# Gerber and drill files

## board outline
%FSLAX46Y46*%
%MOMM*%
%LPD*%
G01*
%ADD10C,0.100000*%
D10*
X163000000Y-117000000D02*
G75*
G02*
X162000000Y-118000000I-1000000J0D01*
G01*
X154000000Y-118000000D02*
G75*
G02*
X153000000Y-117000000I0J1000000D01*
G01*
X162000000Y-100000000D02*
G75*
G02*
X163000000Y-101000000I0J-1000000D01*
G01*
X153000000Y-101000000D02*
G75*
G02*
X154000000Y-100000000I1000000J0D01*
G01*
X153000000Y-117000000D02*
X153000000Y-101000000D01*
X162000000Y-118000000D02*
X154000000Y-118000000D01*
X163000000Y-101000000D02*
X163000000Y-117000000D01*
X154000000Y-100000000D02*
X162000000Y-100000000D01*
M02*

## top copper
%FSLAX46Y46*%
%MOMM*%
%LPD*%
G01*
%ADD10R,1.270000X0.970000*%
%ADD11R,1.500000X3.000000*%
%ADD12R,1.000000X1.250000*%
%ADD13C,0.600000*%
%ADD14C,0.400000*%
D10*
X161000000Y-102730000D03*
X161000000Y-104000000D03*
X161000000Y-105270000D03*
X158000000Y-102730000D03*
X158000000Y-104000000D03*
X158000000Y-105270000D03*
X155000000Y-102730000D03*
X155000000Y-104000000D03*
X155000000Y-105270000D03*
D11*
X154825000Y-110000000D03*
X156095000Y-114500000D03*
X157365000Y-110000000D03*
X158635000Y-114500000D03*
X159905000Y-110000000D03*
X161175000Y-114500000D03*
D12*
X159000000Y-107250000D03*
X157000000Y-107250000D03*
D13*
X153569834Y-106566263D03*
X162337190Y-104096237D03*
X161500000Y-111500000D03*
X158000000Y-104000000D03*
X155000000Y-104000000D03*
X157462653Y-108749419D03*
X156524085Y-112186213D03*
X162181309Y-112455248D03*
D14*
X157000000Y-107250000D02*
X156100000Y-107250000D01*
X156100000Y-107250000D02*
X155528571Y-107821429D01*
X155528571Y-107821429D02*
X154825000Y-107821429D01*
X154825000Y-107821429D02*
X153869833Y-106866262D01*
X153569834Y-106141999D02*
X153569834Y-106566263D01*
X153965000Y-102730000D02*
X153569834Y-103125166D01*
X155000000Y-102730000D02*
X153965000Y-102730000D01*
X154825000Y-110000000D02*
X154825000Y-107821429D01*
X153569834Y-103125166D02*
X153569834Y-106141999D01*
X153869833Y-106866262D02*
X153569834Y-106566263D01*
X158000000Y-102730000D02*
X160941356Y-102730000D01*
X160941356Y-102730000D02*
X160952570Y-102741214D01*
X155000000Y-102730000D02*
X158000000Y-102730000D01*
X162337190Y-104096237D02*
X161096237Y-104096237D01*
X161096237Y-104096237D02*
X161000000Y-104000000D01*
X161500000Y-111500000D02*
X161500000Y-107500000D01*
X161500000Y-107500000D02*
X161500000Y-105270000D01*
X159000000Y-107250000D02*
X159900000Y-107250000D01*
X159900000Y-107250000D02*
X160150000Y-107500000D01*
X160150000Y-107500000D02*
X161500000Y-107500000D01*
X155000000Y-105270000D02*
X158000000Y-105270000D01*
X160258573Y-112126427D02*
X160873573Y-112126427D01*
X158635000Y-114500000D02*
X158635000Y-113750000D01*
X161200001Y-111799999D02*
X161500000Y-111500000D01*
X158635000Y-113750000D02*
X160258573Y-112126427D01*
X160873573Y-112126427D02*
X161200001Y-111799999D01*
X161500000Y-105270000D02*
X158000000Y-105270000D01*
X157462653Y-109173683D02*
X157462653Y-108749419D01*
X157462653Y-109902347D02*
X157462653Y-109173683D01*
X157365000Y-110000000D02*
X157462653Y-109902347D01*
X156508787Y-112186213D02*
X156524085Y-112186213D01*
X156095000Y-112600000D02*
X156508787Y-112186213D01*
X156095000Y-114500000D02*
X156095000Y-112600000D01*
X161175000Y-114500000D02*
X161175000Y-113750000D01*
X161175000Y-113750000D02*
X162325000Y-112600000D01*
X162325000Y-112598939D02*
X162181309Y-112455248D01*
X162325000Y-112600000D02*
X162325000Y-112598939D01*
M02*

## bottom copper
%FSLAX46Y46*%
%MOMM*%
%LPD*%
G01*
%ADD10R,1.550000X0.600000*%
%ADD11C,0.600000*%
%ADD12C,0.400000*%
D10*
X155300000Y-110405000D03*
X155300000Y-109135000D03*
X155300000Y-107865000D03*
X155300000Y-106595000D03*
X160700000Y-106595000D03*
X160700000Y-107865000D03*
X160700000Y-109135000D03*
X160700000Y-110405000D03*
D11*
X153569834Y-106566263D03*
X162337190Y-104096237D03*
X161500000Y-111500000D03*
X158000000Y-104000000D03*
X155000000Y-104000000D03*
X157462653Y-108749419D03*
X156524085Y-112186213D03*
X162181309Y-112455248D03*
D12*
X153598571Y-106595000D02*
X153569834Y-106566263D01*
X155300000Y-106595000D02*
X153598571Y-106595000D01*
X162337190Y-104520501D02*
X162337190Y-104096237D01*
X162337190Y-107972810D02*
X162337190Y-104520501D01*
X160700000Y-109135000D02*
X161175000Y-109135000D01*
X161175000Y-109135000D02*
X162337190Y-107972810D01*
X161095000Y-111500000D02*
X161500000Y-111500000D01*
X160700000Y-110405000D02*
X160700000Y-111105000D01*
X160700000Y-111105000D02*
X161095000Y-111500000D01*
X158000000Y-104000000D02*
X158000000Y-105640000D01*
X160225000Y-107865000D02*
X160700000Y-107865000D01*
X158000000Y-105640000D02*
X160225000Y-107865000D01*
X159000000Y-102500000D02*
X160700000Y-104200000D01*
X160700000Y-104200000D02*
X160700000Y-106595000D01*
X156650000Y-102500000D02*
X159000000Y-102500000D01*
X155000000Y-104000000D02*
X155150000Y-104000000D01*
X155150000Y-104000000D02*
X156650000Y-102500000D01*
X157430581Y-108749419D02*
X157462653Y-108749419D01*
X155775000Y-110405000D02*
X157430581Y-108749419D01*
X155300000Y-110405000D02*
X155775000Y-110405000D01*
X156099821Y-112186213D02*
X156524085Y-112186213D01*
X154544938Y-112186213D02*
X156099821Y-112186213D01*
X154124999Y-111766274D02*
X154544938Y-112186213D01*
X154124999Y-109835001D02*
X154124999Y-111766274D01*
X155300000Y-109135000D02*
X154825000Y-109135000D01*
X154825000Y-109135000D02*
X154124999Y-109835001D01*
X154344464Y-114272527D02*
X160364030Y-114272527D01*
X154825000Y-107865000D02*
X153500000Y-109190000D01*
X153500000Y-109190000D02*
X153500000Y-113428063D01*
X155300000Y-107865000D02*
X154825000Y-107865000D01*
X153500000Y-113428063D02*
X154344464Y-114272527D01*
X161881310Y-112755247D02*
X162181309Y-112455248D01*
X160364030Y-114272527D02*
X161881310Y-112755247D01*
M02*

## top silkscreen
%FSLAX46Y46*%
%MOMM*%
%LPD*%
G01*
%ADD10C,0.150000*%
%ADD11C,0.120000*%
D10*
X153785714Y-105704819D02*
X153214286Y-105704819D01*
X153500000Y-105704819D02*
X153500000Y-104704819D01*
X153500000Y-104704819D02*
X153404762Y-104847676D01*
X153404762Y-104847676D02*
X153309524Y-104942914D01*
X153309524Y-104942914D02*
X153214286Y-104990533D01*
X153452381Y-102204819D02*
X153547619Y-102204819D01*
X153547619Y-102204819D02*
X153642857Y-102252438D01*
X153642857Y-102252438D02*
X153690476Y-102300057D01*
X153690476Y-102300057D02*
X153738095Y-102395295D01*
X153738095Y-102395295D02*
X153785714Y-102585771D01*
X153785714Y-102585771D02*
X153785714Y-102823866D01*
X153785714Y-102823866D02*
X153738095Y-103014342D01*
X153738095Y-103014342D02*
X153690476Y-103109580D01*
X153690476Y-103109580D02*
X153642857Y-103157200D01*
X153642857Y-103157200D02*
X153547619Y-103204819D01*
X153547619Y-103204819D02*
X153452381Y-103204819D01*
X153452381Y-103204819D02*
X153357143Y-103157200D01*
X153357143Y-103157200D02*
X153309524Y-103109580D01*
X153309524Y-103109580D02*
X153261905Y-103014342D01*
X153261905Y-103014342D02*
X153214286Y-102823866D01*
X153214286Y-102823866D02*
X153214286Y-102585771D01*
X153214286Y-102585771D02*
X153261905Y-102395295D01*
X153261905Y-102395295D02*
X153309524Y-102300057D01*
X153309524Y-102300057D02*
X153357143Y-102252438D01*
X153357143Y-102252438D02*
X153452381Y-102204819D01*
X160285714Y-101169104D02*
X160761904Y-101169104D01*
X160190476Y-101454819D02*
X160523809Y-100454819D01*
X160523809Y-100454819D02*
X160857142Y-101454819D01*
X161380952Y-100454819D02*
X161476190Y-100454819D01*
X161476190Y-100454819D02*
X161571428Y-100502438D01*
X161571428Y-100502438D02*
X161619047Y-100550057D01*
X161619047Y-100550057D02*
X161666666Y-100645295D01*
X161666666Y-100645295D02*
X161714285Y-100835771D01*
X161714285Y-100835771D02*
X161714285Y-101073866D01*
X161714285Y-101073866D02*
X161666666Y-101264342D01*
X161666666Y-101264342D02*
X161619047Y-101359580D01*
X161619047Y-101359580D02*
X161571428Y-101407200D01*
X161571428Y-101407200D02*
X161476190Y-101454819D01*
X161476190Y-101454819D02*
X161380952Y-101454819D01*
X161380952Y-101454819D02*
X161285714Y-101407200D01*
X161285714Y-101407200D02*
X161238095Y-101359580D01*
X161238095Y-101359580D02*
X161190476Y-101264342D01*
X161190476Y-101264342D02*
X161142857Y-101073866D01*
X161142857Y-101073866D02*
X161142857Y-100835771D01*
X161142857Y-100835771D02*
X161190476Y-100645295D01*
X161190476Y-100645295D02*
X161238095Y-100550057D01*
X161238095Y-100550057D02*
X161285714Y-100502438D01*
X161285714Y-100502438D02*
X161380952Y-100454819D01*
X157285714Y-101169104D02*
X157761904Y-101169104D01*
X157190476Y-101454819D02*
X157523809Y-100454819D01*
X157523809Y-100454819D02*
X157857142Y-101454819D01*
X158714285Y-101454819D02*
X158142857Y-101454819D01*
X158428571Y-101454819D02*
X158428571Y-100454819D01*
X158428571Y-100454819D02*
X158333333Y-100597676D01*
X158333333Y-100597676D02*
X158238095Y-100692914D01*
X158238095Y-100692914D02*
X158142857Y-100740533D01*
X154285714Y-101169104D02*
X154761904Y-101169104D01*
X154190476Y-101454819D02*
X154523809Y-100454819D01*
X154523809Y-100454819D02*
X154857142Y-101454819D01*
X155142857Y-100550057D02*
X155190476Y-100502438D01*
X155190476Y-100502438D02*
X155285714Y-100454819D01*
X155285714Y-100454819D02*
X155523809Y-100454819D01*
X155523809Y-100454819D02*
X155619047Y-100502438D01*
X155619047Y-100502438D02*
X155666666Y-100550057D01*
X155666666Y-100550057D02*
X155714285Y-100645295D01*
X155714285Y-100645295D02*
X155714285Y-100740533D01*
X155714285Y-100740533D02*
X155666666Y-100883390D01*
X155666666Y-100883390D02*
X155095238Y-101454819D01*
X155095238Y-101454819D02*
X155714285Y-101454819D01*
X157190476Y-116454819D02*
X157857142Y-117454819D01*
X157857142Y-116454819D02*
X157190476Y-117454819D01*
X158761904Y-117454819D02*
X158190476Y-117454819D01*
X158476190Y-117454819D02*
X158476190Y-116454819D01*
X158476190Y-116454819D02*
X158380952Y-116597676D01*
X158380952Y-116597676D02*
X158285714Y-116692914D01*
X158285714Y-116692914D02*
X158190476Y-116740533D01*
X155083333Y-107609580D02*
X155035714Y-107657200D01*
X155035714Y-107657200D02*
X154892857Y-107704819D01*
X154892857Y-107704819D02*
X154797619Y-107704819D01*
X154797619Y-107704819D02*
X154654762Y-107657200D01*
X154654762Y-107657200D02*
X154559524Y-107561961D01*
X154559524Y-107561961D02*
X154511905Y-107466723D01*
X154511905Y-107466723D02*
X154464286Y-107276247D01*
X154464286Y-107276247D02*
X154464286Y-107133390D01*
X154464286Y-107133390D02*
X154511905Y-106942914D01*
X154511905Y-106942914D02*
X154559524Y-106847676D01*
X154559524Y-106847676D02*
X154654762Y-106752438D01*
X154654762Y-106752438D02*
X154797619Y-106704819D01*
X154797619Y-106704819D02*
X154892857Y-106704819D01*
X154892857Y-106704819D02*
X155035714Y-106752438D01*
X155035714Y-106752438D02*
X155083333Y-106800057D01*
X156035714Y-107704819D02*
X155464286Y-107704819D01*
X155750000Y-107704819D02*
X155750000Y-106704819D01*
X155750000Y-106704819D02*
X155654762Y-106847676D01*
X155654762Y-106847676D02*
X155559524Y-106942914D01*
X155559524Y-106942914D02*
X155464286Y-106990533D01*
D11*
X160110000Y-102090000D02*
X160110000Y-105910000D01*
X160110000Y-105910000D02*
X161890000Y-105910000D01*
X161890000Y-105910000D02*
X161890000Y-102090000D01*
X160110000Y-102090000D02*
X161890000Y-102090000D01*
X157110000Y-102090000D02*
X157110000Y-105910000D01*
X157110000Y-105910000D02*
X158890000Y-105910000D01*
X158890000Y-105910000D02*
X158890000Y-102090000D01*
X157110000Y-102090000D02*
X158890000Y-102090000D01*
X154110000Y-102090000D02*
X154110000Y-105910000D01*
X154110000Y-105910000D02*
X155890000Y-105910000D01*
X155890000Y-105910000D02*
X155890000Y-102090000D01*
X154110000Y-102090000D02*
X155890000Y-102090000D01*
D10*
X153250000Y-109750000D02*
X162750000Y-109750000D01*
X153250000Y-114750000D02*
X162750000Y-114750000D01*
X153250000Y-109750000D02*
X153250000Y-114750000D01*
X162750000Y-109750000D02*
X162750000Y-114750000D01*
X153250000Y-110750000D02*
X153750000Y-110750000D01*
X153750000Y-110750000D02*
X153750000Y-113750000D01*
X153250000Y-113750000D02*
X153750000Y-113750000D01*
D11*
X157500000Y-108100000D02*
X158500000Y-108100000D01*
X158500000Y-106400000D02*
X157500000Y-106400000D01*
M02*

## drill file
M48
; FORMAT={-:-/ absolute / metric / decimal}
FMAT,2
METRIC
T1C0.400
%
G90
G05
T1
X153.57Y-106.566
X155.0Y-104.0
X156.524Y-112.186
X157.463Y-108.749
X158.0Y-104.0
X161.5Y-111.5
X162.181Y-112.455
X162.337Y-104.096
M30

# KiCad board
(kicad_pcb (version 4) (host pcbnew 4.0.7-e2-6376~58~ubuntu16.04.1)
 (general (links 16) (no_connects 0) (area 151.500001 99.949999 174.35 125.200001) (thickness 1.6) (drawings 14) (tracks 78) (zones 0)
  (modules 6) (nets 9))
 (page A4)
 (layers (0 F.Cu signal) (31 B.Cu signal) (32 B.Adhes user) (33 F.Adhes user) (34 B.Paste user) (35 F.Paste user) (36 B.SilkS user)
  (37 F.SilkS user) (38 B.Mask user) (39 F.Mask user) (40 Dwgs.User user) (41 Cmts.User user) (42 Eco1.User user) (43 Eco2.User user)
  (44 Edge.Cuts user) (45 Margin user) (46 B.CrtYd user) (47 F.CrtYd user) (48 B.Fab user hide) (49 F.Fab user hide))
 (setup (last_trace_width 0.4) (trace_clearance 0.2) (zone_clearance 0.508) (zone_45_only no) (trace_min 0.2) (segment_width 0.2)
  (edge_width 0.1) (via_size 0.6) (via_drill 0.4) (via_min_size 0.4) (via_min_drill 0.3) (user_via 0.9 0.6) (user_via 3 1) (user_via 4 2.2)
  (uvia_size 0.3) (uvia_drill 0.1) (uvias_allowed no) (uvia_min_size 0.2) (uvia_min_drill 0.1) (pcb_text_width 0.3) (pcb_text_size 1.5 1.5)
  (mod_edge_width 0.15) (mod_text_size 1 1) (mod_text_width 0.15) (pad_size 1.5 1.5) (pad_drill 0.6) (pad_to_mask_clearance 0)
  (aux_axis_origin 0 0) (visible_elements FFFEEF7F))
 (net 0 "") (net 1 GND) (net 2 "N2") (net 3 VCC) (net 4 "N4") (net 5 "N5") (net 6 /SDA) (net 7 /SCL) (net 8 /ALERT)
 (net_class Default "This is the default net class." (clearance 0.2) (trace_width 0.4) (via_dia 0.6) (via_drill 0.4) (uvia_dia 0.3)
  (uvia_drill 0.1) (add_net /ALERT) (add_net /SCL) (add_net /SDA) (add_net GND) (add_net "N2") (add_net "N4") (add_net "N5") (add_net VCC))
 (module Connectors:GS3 (layer F.Cu) (at 161 104)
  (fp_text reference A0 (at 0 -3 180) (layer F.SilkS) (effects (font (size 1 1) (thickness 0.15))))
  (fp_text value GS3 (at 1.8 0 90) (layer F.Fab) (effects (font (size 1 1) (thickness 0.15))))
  (fp_line (start -0.89 -1.91) (end -0.89 1.91) (layer F.SilkS) (width 0.12))
  (fp_line (start -0.89 1.91) (end 0.89 1.91) (layer F.SilkS) (width 0.12))
  (fp_line (start 0.89 1.91) (end 0.89 -1.91) (layer F.SilkS) (width 0.12))
  (fp_line (start -0.89 -1.91) (end 0.89 -1.91) (layer F.SilkS) (width 0.12))
  (pad 1 smd rect (at 0 -1.27) (size 1.27 0.97) (layers F.Cu F.Paste F.Mask) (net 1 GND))
  (pad 2 smd rect (at 0 0) (size 1.27 0.97) (layers F.Cu F.Paste F.Mask) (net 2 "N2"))
  (pad 3 smd rect (at 0 1.27) (size 1.27 0.97) (layers F.Cu F.Paste F.Mask) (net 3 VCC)))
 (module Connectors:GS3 (layer F.Cu) (at 158 104)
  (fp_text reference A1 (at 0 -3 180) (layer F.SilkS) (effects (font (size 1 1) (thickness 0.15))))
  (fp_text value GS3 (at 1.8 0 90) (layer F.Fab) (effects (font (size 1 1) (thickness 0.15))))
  (fp_line (start -0.89 -1.91) (end -0.89 1.91) (layer F.SilkS) (width 0.12))
  (fp_line (start -0.89 1.91) (end 0.89 1.91) (layer F.SilkS) (width 0.12))
  (fp_line (start 0.89 1.91) (end 0.89 -1.91) (layer F.SilkS) (width 0.12))
  (fp_line (start -0.89 -1.91) (end 0.89 -1.91) (layer F.SilkS) (width 0.12))
  (pad 1 smd rect (at 0 -1.27) (size 1.27 0.97) (layers F.Cu F.Paste F.Mask) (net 1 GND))
  (pad 2 smd rect (at 0 0) (size 1.27 0.97) (layers F.Cu F.Paste F.Mask) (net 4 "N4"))
  (pad 3 smd rect (at 0 1.27) (size 1.27 0.97) (layers F.Cu F.Paste F.Mask) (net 3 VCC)))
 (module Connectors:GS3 (layer F.Cu) (at 155 104)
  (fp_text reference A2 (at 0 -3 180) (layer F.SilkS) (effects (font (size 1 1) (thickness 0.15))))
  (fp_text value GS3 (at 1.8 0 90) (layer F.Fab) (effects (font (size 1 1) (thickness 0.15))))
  (fp_line (start -0.89 -1.91) (end -0.89 1.91) (layer F.SilkS) (width 0.12))
  (fp_line (start -0.89 1.91) (end 0.89 1.91) (layer F.SilkS) (width 0.12))
  (fp_line (start 0.89 1.91) (end 0.89 -1.91) (layer F.SilkS) (width 0.12))
  (fp_line (start -0.89 -1.91) (end 0.89 -1.91) (layer F.SilkS) (width 0.12))
  (pad 1 smd rect (at 0 -1.27) (size 1.27 0.97) (layers F.Cu F.Paste F.Mask) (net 1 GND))
  (pad 2 smd rect (at 0 0) (size 1.27 0.97) (layers F.Cu F.Paste F.Mask) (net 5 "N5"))
  (pad 3 smd rect (at 0 1.27) (size 1.27 0.97) (layers F.Cu F.Paste F.Mask) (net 3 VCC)))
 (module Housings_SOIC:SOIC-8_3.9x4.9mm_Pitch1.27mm (layer B.Cu) (at 158 108.5)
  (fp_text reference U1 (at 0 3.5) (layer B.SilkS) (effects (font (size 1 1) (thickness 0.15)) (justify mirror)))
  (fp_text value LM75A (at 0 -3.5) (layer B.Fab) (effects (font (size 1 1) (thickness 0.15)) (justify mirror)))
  (pad 1 smd rect (at -2.7 1.905) (size 1.55 0.6) (layers B.Cu B.Paste B.Mask) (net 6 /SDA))
  (pad 2 smd rect (at -2.7 0.635) (size 1.55 0.6) (layers B.Cu B.Paste B.Mask) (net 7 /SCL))
  (pad 3 smd rect (at -2.7 -0.635) (size 1.55 0.6) (layers B.Cu B.Paste B.Mask) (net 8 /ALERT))
  (pad 4 smd rect (at -2.7 -1.905) (size 1.55 0.6) (layers B.Cu B.Paste B.Mask) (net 1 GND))
  (pad 5 smd rect (at 2.7 -1.905) (size 1.55 0.6) (layers B.Cu B.Paste B.Mask) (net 5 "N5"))
  (pad 6 smd rect (at 2.7 -0.635) (size 1.55 0.6) (layers B.Cu B.Paste B.Mask) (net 4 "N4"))
  (pad 7 smd rect (at 2.7 0.635) (size 1.55 0.6) (layers B.Cu B.Paste B.Mask) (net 2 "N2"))
  (pad 8 smd rect (at 2.7 1.905) (size 1.55 0.6) (layers B.Cu B.Paste B.Mask) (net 3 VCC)))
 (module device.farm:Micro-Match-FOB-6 (layer F.Cu) (at 158 112.25)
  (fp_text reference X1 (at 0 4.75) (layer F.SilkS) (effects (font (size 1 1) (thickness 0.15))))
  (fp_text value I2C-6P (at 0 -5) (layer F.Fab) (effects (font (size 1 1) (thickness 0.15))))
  (fp_line (start -4.75 -2.5) (end 4.75 -2.5) (layer F.SilkS) (width 0.15))
  (fp_line (start -4.75 2.5) (end 4.75 2.5) (layer F.SilkS) (width 0.15))
  (fp_line (start -4.75 -2.5) (end -4.75 2.5) (layer F.SilkS) (width 0.15))
  (fp_line (start 4.75 -2.5) (end 4.75 2.5) (layer F.SilkS) (width 0.15))
  (fp_line (start -4.75 -1.5) (end -4.25 -1.5) (layer F.SilkS) (width 0.15))
  (fp_line (start -4.25 -1.5) (end -4.25 1.5) (layer F.SilkS) (width 0.15))
  (fp_line (start -4.75 1.5) (end -4.25 1.5) (layer F.SilkS) (width 0.15))
  (pad 1 smd rect (at -3.175 -2.25) (size 1.5 3) (layers F.Cu F.Paste F.Mask) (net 1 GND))
  (pad 2 smd rect (at -1.905 2.25) (size 1.5 3) (layers F.Cu F.Paste F.Mask) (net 7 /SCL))
  (pad 3 smd rect (at -0.635 -2.25) (size 1.5 3) (layers F.Cu F.Paste F.Mask) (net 6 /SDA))
  (pad 4 smd rect (at 0.635 2.25) (size 1.5 3) (layers F.Cu F.Paste F.Mask) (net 3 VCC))
  (pad 5 smd rect (at 1.905 -2.25) (size 1.5 3) (layers F.Cu F.Paste F.Mask))
  (pad 6 smd rect (at 3.175 2.25) (size 1.5 3) (layers F.Cu F.Paste F.Mask) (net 8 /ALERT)))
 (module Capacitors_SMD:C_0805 (layer F.Cu) (at 158 107.25 180)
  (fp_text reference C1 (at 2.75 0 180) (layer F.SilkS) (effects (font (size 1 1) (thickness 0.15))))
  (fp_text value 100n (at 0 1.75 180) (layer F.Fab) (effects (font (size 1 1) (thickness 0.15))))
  (fp_line (start 0.5 -0.85) (end -0.5 -0.85) (layer F.SilkS) (width 0.12))
  (fp_line (start -0.5 0.85) (end 0.5 0.85) (layer F.SilkS) (width 0.12))
  (pad 1 smd rect (at -1 0 180) (size 1 1.25) (layers F.Cu F.Paste F.Mask) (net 3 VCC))
  (pad 2 smd rect (at 1 0 180) (size 1 1.25) (layers F.Cu F.Paste F.Mask) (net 1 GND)))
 (gr_arc (start 162 117) (end 163 117) (angle 90) (layer Edge.Cuts) (width 0.1))
 (gr_arc (start 154 117) (end 154 118) (angle 90) (layer Edge.Cuts) (width 0.1))
 (gr_arc (start 162 101) (end 162 100) (angle 90) (layer Edge.Cuts) (width 0.1))
 (gr_arc (start 154 101) (end 153 101) (angle 90) (layer Edge.Cuts) (width 0.1))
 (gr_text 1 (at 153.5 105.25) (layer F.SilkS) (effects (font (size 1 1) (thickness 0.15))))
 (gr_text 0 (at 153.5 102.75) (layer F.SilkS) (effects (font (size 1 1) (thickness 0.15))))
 (gr_line (start 153 117) (end 153 101) (layer Edge.Cuts) (width 0.1))
 (gr_line (start 162 118) (end 154 118) (layer Edge.Cuts) (width 0.1))
 (gr_line (start 163 101) (end 163 117) (layer Edge.Cuts) (width 0.1))
 (gr_line (start 154 100) (end 162 100) (layer Edge.Cuts) (width 0.1))
 (segment (start 157 107.25) (end 156.1 107.25) (width 0.4) (layer F.Cu) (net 1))
 (segment (start 156.1 107.25) (end 155.528571 107.821429) (width 0.4) (layer F.Cu) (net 1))
 (segment (start 155.528571 107.821429) (end 154.825 107.821429) (width 0.4) (layer F.Cu) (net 1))
 (segment (start 154.825 107.821429) (end 153.869833 106.866262) (width 0.4) (layer F.Cu) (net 1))
 (segment (start 153.569834 106.141999) (end 153.569834 106.566263) (width 0.4) (layer F.Cu) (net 1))
 (segment (start 153.965 102.73) (end 153.569834 103.125166) (width 0.4) (layer F.Cu) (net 1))
 (segment (start 155 102.73) (end 153.965 102.73) (width 0.4) (layer F.Cu) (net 1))
 (segment (start 153.598571 106.595) (end 153.569834 106.566263) (width 0.4) (layer B.Cu) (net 1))
 (segment (start 155.3 106.595) (end 153.598571 106.595) (width 0.4) (layer B.Cu) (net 1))
 (segment (start 154.825 110) (end 154.825 107.821429) (width 0.4) (layer F.Cu) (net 1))
 (segment (start 153.569834 103.125166) (end 153.569834 106.141999) (width 0.4) (layer F.Cu) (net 1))
 (segment (start 153.869833 106.866262) (end 153.569834 106.566263) (width 0.4) (layer F.Cu) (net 1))
 (via (at 153.569834 106.566263) (size 0.6) (drill 0.4) (layers F.Cu B.Cu) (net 1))
 (segment (start 158 102.73) (end 160.941356 102.73) (width 0.4) (layer F.Cu) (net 1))
 (segment (start 160.941356 102.73) (end 160.95257 102.741214) (width 0.4) (layer F.Cu) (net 1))
 (segment (start 155 102.73) (end 158 102.73) (width 0.4) (layer F.Cu) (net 1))
 (segment (start 162.33719 104.096237) (end 161.096237 104.096237) (width 0.4) (layer F.Cu) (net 2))
 (segment (start 161.096237 104.096237) (end 161 104) (width 0.4) (layer F.Cu) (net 2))
 (segment (start 162.33719 104.520501) (end 162.33719 104.096237) (width 0.4) (layer B.Cu) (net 2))
 (segment (start 162.33719 107.97281) (end 162.33719 104.520501) (width 0.4) (layer B.Cu) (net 2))
 (segment (start 160.7 109.135) (end 161.175 109.135) (width 0.4) (layer B.Cu) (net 2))
 (segment (start 161.175 109.135) (end 162.33719 107.97281) (width 0.4) (layer B.Cu) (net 2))
 (via (at 162.33719 104.096237) (size 0.6) (drill 0.4) (layers F.Cu B.Cu) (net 2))
 (segment (start 161.5 111.5) (end 161.5 107.5) (width 0.4) (layer F.Cu) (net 3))
 (segment (start 161.5 107.5) (end 161.5 105.27) (width 0.4) (layer F.Cu) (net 3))
 (segment (start 159 107.25) (end 159.9 107.25) (width 0.4) (layer F.Cu) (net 3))
 (segment (start 159.9 107.25) (end 160.15 107.5) (width 0.4) (layer F.Cu) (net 3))
 (segment (start 160.15 107.5) (end 161.5 107.5) (width 0.4) (layer F.Cu) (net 3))
 (segment (start 155 105.27) (end 158 105.27) (width 0.4) (layer F.Cu) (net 3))
 (segment (start 160.258573 112.126427) (end 160.873573 112.126427) (width 0.4) (layer F.Cu) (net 3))
 (segment (start 158.635 114.5) (end 158.635 113.75) (width 0.4) (layer F.Cu) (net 3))
 (segment (start 161.200001 111.799999) (end 161.5 111.5) (width 0.4) (layer F.Cu) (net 3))
 (segment (start 158.635 113.75) (end 160.258573 112.126427) (width 0.4) (layer F.Cu) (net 3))
 (segment (start 160.873573 112.126427) (end 161.200001 111.799999) (width 0.4) (layer F.Cu) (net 3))
 (segment (start 161.5 105.27) (end 158 105.27) (width 0.4) (layer F.Cu) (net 3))
 (via (at 161.5 111.5) (size 0.6) (drill 0.4) (layers F.Cu B.Cu) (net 3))
 (segment (start 161.095 111.5) (end 161.5 111.5) (width 0.4) (layer B.Cu) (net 3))
 (segment (start 160.7 110.405) (end 160.7 111.105) (width 0.4) (layer B.Cu) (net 3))
 (segment (start 160.7 111.105) (end 161.095 111.5) (width 0.4) (layer B.Cu) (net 3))
 (segment (start 158 104) (end 158 105.64) (width 0.4) (layer B.Cu) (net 4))
 (segment (start 160.225 107.865) (end 160.7 107.865) (width 0.4) (layer B.Cu) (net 4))
 (segment (start 158 105.64) (end 160.225 107.865) (width 0.4) (layer B.Cu) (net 4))
 (via (at 158 104) (size 0.6) (drill 0.4) (layers F.Cu B.Cu) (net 4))
 (segment (start 159 102.5) (end 160.7 104.2) (width 0.4) (layer B.Cu) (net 5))
 (segment (start 160.7 104.2) (end 160.7 106.595) (width 0.4) (layer B.Cu) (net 5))
 (segment (start 156.65 102.5) (end 159 102.5) (width 0.4) (layer B.Cu) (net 5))
 (segment (start 155 104) (end 155.15 104) (width 0.4) (layer B.Cu) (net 5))
 (segment (start 155.15 104) (end 156.65 102.5) (width 0.4) (layer B.Cu) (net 5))
 (via (at 155 104) (size 0.6) (drill 0.4) (layers F.Cu B.Cu) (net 5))
 (segment (start 157.430581 108.749419) (end 157.462653 108.749419) (width 0.4) (layer B.Cu) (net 6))
 (segment (start 155.775 110.405) (end 157.430581 108.749419) (width 0.4) (layer B.Cu) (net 6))
 (segment (start 155.3 110.405) (end 155.775 110.405) (width 0.4) (layer B.Cu) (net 6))
 (segment (start 157.462653 109.173683) (end 157.462653 108.749419) (width 0.4) (layer F.Cu) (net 6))
 (segment (start 157.462653 109.902347) (end 157.462653 109.173683) (width 0.4) (layer F.Cu) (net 6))
 (segment (start 157.365 110) (end 157.462653 109.902347) (width 0.4) (layer F.Cu) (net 6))
 (via (at 157.462653 108.749419) (size 0.6) (drill 0.4) (layers F.Cu B.Cu) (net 6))
 (segment (start 156.508787 112.186213) (end 156.524085 112.186213) (width 0.4) (layer F.Cu) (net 7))
 (segment (start 156.095 112.6) (end 156.508787 112.186213) (width 0.4) (layer F.Cu) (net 7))
 (segment (start 156.095 114.5) (end 156.095 112.6) (width 0.4) (layer F.Cu) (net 7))
 (segment (start 156.099821 112.186213) (end 156.524085 112.186213) (width 0.4) (layer B.Cu) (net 7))
 (segment (start 154.544938 112.186213) (end 156.099821 112.186213) (width 0.4) (layer B.Cu) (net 7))
 (segment (start 154.124999 111.766274) (end 154.544938 112.186213) (width 0.4) (layer B.Cu) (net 7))
 (segment (start 154.124999 109.835001) (end 154.124999 111.766274) (width 0.4) (layer B.Cu) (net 7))
 (segment (start 155.3 109.135) (end 154.825 109.135) (width 0.4) (layer B.Cu) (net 7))
 (segment (start 154.825 109.135) (end 154.124999 109.835001) (width 0.4) (layer B.Cu) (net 7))
 (via (at 156.524085 112.186213) (size 0.6) (drill 0.4) (layers F.Cu B.Cu) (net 7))
 (segment (start 161.175 114.5) (end 161.175 113.75) (width 0.4) (layer F.Cu) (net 8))
 (segment (start 161.175 113.75) (end 162.325 112.6) (width 0.4) (layer F.Cu) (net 8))
 (segment (start 154.344464 114.272527) (end 160.36403 114.272527) (width 0.4) (layer B.Cu) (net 8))
 (segment (start 154.825 107.865) (end 153.5 109.19) (width 0.4) (layer B.Cu) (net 8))
 (segment (start 153.5 109.19) (end 153.5 113.428063) (width 0.4) (layer B.Cu) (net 8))
 (segment (start 162.325 112.598939) (end 162.181309 112.455248) (width 0.4) (layer F.Cu) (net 8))
 (segment (start 155.3 107.865) (end 154.825 107.865) (width 0.4) (layer B.Cu) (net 8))
 (segment (start 153.5 113.428063) (end 154.344464 114.272527) (width 0.4) (layer B.Cu) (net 8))
 (segment (start 161.88131 112.755247) (end 162.181309 112.455248) (width 0.4) (layer B.Cu) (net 8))
 (segment (start 160.36403 114.272527) (end 161.88131 112.755247) (width 0.4) (layer B.Cu) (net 8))
 (via (at 162.181309 112.455248) (size 0.6) (drill 0.4) (layers F.Cu B.Cu) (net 8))
 (segment (start 162.325 112.6) (end 162.325 112.598939) (width 0.4) (layer F.Cu) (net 8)))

